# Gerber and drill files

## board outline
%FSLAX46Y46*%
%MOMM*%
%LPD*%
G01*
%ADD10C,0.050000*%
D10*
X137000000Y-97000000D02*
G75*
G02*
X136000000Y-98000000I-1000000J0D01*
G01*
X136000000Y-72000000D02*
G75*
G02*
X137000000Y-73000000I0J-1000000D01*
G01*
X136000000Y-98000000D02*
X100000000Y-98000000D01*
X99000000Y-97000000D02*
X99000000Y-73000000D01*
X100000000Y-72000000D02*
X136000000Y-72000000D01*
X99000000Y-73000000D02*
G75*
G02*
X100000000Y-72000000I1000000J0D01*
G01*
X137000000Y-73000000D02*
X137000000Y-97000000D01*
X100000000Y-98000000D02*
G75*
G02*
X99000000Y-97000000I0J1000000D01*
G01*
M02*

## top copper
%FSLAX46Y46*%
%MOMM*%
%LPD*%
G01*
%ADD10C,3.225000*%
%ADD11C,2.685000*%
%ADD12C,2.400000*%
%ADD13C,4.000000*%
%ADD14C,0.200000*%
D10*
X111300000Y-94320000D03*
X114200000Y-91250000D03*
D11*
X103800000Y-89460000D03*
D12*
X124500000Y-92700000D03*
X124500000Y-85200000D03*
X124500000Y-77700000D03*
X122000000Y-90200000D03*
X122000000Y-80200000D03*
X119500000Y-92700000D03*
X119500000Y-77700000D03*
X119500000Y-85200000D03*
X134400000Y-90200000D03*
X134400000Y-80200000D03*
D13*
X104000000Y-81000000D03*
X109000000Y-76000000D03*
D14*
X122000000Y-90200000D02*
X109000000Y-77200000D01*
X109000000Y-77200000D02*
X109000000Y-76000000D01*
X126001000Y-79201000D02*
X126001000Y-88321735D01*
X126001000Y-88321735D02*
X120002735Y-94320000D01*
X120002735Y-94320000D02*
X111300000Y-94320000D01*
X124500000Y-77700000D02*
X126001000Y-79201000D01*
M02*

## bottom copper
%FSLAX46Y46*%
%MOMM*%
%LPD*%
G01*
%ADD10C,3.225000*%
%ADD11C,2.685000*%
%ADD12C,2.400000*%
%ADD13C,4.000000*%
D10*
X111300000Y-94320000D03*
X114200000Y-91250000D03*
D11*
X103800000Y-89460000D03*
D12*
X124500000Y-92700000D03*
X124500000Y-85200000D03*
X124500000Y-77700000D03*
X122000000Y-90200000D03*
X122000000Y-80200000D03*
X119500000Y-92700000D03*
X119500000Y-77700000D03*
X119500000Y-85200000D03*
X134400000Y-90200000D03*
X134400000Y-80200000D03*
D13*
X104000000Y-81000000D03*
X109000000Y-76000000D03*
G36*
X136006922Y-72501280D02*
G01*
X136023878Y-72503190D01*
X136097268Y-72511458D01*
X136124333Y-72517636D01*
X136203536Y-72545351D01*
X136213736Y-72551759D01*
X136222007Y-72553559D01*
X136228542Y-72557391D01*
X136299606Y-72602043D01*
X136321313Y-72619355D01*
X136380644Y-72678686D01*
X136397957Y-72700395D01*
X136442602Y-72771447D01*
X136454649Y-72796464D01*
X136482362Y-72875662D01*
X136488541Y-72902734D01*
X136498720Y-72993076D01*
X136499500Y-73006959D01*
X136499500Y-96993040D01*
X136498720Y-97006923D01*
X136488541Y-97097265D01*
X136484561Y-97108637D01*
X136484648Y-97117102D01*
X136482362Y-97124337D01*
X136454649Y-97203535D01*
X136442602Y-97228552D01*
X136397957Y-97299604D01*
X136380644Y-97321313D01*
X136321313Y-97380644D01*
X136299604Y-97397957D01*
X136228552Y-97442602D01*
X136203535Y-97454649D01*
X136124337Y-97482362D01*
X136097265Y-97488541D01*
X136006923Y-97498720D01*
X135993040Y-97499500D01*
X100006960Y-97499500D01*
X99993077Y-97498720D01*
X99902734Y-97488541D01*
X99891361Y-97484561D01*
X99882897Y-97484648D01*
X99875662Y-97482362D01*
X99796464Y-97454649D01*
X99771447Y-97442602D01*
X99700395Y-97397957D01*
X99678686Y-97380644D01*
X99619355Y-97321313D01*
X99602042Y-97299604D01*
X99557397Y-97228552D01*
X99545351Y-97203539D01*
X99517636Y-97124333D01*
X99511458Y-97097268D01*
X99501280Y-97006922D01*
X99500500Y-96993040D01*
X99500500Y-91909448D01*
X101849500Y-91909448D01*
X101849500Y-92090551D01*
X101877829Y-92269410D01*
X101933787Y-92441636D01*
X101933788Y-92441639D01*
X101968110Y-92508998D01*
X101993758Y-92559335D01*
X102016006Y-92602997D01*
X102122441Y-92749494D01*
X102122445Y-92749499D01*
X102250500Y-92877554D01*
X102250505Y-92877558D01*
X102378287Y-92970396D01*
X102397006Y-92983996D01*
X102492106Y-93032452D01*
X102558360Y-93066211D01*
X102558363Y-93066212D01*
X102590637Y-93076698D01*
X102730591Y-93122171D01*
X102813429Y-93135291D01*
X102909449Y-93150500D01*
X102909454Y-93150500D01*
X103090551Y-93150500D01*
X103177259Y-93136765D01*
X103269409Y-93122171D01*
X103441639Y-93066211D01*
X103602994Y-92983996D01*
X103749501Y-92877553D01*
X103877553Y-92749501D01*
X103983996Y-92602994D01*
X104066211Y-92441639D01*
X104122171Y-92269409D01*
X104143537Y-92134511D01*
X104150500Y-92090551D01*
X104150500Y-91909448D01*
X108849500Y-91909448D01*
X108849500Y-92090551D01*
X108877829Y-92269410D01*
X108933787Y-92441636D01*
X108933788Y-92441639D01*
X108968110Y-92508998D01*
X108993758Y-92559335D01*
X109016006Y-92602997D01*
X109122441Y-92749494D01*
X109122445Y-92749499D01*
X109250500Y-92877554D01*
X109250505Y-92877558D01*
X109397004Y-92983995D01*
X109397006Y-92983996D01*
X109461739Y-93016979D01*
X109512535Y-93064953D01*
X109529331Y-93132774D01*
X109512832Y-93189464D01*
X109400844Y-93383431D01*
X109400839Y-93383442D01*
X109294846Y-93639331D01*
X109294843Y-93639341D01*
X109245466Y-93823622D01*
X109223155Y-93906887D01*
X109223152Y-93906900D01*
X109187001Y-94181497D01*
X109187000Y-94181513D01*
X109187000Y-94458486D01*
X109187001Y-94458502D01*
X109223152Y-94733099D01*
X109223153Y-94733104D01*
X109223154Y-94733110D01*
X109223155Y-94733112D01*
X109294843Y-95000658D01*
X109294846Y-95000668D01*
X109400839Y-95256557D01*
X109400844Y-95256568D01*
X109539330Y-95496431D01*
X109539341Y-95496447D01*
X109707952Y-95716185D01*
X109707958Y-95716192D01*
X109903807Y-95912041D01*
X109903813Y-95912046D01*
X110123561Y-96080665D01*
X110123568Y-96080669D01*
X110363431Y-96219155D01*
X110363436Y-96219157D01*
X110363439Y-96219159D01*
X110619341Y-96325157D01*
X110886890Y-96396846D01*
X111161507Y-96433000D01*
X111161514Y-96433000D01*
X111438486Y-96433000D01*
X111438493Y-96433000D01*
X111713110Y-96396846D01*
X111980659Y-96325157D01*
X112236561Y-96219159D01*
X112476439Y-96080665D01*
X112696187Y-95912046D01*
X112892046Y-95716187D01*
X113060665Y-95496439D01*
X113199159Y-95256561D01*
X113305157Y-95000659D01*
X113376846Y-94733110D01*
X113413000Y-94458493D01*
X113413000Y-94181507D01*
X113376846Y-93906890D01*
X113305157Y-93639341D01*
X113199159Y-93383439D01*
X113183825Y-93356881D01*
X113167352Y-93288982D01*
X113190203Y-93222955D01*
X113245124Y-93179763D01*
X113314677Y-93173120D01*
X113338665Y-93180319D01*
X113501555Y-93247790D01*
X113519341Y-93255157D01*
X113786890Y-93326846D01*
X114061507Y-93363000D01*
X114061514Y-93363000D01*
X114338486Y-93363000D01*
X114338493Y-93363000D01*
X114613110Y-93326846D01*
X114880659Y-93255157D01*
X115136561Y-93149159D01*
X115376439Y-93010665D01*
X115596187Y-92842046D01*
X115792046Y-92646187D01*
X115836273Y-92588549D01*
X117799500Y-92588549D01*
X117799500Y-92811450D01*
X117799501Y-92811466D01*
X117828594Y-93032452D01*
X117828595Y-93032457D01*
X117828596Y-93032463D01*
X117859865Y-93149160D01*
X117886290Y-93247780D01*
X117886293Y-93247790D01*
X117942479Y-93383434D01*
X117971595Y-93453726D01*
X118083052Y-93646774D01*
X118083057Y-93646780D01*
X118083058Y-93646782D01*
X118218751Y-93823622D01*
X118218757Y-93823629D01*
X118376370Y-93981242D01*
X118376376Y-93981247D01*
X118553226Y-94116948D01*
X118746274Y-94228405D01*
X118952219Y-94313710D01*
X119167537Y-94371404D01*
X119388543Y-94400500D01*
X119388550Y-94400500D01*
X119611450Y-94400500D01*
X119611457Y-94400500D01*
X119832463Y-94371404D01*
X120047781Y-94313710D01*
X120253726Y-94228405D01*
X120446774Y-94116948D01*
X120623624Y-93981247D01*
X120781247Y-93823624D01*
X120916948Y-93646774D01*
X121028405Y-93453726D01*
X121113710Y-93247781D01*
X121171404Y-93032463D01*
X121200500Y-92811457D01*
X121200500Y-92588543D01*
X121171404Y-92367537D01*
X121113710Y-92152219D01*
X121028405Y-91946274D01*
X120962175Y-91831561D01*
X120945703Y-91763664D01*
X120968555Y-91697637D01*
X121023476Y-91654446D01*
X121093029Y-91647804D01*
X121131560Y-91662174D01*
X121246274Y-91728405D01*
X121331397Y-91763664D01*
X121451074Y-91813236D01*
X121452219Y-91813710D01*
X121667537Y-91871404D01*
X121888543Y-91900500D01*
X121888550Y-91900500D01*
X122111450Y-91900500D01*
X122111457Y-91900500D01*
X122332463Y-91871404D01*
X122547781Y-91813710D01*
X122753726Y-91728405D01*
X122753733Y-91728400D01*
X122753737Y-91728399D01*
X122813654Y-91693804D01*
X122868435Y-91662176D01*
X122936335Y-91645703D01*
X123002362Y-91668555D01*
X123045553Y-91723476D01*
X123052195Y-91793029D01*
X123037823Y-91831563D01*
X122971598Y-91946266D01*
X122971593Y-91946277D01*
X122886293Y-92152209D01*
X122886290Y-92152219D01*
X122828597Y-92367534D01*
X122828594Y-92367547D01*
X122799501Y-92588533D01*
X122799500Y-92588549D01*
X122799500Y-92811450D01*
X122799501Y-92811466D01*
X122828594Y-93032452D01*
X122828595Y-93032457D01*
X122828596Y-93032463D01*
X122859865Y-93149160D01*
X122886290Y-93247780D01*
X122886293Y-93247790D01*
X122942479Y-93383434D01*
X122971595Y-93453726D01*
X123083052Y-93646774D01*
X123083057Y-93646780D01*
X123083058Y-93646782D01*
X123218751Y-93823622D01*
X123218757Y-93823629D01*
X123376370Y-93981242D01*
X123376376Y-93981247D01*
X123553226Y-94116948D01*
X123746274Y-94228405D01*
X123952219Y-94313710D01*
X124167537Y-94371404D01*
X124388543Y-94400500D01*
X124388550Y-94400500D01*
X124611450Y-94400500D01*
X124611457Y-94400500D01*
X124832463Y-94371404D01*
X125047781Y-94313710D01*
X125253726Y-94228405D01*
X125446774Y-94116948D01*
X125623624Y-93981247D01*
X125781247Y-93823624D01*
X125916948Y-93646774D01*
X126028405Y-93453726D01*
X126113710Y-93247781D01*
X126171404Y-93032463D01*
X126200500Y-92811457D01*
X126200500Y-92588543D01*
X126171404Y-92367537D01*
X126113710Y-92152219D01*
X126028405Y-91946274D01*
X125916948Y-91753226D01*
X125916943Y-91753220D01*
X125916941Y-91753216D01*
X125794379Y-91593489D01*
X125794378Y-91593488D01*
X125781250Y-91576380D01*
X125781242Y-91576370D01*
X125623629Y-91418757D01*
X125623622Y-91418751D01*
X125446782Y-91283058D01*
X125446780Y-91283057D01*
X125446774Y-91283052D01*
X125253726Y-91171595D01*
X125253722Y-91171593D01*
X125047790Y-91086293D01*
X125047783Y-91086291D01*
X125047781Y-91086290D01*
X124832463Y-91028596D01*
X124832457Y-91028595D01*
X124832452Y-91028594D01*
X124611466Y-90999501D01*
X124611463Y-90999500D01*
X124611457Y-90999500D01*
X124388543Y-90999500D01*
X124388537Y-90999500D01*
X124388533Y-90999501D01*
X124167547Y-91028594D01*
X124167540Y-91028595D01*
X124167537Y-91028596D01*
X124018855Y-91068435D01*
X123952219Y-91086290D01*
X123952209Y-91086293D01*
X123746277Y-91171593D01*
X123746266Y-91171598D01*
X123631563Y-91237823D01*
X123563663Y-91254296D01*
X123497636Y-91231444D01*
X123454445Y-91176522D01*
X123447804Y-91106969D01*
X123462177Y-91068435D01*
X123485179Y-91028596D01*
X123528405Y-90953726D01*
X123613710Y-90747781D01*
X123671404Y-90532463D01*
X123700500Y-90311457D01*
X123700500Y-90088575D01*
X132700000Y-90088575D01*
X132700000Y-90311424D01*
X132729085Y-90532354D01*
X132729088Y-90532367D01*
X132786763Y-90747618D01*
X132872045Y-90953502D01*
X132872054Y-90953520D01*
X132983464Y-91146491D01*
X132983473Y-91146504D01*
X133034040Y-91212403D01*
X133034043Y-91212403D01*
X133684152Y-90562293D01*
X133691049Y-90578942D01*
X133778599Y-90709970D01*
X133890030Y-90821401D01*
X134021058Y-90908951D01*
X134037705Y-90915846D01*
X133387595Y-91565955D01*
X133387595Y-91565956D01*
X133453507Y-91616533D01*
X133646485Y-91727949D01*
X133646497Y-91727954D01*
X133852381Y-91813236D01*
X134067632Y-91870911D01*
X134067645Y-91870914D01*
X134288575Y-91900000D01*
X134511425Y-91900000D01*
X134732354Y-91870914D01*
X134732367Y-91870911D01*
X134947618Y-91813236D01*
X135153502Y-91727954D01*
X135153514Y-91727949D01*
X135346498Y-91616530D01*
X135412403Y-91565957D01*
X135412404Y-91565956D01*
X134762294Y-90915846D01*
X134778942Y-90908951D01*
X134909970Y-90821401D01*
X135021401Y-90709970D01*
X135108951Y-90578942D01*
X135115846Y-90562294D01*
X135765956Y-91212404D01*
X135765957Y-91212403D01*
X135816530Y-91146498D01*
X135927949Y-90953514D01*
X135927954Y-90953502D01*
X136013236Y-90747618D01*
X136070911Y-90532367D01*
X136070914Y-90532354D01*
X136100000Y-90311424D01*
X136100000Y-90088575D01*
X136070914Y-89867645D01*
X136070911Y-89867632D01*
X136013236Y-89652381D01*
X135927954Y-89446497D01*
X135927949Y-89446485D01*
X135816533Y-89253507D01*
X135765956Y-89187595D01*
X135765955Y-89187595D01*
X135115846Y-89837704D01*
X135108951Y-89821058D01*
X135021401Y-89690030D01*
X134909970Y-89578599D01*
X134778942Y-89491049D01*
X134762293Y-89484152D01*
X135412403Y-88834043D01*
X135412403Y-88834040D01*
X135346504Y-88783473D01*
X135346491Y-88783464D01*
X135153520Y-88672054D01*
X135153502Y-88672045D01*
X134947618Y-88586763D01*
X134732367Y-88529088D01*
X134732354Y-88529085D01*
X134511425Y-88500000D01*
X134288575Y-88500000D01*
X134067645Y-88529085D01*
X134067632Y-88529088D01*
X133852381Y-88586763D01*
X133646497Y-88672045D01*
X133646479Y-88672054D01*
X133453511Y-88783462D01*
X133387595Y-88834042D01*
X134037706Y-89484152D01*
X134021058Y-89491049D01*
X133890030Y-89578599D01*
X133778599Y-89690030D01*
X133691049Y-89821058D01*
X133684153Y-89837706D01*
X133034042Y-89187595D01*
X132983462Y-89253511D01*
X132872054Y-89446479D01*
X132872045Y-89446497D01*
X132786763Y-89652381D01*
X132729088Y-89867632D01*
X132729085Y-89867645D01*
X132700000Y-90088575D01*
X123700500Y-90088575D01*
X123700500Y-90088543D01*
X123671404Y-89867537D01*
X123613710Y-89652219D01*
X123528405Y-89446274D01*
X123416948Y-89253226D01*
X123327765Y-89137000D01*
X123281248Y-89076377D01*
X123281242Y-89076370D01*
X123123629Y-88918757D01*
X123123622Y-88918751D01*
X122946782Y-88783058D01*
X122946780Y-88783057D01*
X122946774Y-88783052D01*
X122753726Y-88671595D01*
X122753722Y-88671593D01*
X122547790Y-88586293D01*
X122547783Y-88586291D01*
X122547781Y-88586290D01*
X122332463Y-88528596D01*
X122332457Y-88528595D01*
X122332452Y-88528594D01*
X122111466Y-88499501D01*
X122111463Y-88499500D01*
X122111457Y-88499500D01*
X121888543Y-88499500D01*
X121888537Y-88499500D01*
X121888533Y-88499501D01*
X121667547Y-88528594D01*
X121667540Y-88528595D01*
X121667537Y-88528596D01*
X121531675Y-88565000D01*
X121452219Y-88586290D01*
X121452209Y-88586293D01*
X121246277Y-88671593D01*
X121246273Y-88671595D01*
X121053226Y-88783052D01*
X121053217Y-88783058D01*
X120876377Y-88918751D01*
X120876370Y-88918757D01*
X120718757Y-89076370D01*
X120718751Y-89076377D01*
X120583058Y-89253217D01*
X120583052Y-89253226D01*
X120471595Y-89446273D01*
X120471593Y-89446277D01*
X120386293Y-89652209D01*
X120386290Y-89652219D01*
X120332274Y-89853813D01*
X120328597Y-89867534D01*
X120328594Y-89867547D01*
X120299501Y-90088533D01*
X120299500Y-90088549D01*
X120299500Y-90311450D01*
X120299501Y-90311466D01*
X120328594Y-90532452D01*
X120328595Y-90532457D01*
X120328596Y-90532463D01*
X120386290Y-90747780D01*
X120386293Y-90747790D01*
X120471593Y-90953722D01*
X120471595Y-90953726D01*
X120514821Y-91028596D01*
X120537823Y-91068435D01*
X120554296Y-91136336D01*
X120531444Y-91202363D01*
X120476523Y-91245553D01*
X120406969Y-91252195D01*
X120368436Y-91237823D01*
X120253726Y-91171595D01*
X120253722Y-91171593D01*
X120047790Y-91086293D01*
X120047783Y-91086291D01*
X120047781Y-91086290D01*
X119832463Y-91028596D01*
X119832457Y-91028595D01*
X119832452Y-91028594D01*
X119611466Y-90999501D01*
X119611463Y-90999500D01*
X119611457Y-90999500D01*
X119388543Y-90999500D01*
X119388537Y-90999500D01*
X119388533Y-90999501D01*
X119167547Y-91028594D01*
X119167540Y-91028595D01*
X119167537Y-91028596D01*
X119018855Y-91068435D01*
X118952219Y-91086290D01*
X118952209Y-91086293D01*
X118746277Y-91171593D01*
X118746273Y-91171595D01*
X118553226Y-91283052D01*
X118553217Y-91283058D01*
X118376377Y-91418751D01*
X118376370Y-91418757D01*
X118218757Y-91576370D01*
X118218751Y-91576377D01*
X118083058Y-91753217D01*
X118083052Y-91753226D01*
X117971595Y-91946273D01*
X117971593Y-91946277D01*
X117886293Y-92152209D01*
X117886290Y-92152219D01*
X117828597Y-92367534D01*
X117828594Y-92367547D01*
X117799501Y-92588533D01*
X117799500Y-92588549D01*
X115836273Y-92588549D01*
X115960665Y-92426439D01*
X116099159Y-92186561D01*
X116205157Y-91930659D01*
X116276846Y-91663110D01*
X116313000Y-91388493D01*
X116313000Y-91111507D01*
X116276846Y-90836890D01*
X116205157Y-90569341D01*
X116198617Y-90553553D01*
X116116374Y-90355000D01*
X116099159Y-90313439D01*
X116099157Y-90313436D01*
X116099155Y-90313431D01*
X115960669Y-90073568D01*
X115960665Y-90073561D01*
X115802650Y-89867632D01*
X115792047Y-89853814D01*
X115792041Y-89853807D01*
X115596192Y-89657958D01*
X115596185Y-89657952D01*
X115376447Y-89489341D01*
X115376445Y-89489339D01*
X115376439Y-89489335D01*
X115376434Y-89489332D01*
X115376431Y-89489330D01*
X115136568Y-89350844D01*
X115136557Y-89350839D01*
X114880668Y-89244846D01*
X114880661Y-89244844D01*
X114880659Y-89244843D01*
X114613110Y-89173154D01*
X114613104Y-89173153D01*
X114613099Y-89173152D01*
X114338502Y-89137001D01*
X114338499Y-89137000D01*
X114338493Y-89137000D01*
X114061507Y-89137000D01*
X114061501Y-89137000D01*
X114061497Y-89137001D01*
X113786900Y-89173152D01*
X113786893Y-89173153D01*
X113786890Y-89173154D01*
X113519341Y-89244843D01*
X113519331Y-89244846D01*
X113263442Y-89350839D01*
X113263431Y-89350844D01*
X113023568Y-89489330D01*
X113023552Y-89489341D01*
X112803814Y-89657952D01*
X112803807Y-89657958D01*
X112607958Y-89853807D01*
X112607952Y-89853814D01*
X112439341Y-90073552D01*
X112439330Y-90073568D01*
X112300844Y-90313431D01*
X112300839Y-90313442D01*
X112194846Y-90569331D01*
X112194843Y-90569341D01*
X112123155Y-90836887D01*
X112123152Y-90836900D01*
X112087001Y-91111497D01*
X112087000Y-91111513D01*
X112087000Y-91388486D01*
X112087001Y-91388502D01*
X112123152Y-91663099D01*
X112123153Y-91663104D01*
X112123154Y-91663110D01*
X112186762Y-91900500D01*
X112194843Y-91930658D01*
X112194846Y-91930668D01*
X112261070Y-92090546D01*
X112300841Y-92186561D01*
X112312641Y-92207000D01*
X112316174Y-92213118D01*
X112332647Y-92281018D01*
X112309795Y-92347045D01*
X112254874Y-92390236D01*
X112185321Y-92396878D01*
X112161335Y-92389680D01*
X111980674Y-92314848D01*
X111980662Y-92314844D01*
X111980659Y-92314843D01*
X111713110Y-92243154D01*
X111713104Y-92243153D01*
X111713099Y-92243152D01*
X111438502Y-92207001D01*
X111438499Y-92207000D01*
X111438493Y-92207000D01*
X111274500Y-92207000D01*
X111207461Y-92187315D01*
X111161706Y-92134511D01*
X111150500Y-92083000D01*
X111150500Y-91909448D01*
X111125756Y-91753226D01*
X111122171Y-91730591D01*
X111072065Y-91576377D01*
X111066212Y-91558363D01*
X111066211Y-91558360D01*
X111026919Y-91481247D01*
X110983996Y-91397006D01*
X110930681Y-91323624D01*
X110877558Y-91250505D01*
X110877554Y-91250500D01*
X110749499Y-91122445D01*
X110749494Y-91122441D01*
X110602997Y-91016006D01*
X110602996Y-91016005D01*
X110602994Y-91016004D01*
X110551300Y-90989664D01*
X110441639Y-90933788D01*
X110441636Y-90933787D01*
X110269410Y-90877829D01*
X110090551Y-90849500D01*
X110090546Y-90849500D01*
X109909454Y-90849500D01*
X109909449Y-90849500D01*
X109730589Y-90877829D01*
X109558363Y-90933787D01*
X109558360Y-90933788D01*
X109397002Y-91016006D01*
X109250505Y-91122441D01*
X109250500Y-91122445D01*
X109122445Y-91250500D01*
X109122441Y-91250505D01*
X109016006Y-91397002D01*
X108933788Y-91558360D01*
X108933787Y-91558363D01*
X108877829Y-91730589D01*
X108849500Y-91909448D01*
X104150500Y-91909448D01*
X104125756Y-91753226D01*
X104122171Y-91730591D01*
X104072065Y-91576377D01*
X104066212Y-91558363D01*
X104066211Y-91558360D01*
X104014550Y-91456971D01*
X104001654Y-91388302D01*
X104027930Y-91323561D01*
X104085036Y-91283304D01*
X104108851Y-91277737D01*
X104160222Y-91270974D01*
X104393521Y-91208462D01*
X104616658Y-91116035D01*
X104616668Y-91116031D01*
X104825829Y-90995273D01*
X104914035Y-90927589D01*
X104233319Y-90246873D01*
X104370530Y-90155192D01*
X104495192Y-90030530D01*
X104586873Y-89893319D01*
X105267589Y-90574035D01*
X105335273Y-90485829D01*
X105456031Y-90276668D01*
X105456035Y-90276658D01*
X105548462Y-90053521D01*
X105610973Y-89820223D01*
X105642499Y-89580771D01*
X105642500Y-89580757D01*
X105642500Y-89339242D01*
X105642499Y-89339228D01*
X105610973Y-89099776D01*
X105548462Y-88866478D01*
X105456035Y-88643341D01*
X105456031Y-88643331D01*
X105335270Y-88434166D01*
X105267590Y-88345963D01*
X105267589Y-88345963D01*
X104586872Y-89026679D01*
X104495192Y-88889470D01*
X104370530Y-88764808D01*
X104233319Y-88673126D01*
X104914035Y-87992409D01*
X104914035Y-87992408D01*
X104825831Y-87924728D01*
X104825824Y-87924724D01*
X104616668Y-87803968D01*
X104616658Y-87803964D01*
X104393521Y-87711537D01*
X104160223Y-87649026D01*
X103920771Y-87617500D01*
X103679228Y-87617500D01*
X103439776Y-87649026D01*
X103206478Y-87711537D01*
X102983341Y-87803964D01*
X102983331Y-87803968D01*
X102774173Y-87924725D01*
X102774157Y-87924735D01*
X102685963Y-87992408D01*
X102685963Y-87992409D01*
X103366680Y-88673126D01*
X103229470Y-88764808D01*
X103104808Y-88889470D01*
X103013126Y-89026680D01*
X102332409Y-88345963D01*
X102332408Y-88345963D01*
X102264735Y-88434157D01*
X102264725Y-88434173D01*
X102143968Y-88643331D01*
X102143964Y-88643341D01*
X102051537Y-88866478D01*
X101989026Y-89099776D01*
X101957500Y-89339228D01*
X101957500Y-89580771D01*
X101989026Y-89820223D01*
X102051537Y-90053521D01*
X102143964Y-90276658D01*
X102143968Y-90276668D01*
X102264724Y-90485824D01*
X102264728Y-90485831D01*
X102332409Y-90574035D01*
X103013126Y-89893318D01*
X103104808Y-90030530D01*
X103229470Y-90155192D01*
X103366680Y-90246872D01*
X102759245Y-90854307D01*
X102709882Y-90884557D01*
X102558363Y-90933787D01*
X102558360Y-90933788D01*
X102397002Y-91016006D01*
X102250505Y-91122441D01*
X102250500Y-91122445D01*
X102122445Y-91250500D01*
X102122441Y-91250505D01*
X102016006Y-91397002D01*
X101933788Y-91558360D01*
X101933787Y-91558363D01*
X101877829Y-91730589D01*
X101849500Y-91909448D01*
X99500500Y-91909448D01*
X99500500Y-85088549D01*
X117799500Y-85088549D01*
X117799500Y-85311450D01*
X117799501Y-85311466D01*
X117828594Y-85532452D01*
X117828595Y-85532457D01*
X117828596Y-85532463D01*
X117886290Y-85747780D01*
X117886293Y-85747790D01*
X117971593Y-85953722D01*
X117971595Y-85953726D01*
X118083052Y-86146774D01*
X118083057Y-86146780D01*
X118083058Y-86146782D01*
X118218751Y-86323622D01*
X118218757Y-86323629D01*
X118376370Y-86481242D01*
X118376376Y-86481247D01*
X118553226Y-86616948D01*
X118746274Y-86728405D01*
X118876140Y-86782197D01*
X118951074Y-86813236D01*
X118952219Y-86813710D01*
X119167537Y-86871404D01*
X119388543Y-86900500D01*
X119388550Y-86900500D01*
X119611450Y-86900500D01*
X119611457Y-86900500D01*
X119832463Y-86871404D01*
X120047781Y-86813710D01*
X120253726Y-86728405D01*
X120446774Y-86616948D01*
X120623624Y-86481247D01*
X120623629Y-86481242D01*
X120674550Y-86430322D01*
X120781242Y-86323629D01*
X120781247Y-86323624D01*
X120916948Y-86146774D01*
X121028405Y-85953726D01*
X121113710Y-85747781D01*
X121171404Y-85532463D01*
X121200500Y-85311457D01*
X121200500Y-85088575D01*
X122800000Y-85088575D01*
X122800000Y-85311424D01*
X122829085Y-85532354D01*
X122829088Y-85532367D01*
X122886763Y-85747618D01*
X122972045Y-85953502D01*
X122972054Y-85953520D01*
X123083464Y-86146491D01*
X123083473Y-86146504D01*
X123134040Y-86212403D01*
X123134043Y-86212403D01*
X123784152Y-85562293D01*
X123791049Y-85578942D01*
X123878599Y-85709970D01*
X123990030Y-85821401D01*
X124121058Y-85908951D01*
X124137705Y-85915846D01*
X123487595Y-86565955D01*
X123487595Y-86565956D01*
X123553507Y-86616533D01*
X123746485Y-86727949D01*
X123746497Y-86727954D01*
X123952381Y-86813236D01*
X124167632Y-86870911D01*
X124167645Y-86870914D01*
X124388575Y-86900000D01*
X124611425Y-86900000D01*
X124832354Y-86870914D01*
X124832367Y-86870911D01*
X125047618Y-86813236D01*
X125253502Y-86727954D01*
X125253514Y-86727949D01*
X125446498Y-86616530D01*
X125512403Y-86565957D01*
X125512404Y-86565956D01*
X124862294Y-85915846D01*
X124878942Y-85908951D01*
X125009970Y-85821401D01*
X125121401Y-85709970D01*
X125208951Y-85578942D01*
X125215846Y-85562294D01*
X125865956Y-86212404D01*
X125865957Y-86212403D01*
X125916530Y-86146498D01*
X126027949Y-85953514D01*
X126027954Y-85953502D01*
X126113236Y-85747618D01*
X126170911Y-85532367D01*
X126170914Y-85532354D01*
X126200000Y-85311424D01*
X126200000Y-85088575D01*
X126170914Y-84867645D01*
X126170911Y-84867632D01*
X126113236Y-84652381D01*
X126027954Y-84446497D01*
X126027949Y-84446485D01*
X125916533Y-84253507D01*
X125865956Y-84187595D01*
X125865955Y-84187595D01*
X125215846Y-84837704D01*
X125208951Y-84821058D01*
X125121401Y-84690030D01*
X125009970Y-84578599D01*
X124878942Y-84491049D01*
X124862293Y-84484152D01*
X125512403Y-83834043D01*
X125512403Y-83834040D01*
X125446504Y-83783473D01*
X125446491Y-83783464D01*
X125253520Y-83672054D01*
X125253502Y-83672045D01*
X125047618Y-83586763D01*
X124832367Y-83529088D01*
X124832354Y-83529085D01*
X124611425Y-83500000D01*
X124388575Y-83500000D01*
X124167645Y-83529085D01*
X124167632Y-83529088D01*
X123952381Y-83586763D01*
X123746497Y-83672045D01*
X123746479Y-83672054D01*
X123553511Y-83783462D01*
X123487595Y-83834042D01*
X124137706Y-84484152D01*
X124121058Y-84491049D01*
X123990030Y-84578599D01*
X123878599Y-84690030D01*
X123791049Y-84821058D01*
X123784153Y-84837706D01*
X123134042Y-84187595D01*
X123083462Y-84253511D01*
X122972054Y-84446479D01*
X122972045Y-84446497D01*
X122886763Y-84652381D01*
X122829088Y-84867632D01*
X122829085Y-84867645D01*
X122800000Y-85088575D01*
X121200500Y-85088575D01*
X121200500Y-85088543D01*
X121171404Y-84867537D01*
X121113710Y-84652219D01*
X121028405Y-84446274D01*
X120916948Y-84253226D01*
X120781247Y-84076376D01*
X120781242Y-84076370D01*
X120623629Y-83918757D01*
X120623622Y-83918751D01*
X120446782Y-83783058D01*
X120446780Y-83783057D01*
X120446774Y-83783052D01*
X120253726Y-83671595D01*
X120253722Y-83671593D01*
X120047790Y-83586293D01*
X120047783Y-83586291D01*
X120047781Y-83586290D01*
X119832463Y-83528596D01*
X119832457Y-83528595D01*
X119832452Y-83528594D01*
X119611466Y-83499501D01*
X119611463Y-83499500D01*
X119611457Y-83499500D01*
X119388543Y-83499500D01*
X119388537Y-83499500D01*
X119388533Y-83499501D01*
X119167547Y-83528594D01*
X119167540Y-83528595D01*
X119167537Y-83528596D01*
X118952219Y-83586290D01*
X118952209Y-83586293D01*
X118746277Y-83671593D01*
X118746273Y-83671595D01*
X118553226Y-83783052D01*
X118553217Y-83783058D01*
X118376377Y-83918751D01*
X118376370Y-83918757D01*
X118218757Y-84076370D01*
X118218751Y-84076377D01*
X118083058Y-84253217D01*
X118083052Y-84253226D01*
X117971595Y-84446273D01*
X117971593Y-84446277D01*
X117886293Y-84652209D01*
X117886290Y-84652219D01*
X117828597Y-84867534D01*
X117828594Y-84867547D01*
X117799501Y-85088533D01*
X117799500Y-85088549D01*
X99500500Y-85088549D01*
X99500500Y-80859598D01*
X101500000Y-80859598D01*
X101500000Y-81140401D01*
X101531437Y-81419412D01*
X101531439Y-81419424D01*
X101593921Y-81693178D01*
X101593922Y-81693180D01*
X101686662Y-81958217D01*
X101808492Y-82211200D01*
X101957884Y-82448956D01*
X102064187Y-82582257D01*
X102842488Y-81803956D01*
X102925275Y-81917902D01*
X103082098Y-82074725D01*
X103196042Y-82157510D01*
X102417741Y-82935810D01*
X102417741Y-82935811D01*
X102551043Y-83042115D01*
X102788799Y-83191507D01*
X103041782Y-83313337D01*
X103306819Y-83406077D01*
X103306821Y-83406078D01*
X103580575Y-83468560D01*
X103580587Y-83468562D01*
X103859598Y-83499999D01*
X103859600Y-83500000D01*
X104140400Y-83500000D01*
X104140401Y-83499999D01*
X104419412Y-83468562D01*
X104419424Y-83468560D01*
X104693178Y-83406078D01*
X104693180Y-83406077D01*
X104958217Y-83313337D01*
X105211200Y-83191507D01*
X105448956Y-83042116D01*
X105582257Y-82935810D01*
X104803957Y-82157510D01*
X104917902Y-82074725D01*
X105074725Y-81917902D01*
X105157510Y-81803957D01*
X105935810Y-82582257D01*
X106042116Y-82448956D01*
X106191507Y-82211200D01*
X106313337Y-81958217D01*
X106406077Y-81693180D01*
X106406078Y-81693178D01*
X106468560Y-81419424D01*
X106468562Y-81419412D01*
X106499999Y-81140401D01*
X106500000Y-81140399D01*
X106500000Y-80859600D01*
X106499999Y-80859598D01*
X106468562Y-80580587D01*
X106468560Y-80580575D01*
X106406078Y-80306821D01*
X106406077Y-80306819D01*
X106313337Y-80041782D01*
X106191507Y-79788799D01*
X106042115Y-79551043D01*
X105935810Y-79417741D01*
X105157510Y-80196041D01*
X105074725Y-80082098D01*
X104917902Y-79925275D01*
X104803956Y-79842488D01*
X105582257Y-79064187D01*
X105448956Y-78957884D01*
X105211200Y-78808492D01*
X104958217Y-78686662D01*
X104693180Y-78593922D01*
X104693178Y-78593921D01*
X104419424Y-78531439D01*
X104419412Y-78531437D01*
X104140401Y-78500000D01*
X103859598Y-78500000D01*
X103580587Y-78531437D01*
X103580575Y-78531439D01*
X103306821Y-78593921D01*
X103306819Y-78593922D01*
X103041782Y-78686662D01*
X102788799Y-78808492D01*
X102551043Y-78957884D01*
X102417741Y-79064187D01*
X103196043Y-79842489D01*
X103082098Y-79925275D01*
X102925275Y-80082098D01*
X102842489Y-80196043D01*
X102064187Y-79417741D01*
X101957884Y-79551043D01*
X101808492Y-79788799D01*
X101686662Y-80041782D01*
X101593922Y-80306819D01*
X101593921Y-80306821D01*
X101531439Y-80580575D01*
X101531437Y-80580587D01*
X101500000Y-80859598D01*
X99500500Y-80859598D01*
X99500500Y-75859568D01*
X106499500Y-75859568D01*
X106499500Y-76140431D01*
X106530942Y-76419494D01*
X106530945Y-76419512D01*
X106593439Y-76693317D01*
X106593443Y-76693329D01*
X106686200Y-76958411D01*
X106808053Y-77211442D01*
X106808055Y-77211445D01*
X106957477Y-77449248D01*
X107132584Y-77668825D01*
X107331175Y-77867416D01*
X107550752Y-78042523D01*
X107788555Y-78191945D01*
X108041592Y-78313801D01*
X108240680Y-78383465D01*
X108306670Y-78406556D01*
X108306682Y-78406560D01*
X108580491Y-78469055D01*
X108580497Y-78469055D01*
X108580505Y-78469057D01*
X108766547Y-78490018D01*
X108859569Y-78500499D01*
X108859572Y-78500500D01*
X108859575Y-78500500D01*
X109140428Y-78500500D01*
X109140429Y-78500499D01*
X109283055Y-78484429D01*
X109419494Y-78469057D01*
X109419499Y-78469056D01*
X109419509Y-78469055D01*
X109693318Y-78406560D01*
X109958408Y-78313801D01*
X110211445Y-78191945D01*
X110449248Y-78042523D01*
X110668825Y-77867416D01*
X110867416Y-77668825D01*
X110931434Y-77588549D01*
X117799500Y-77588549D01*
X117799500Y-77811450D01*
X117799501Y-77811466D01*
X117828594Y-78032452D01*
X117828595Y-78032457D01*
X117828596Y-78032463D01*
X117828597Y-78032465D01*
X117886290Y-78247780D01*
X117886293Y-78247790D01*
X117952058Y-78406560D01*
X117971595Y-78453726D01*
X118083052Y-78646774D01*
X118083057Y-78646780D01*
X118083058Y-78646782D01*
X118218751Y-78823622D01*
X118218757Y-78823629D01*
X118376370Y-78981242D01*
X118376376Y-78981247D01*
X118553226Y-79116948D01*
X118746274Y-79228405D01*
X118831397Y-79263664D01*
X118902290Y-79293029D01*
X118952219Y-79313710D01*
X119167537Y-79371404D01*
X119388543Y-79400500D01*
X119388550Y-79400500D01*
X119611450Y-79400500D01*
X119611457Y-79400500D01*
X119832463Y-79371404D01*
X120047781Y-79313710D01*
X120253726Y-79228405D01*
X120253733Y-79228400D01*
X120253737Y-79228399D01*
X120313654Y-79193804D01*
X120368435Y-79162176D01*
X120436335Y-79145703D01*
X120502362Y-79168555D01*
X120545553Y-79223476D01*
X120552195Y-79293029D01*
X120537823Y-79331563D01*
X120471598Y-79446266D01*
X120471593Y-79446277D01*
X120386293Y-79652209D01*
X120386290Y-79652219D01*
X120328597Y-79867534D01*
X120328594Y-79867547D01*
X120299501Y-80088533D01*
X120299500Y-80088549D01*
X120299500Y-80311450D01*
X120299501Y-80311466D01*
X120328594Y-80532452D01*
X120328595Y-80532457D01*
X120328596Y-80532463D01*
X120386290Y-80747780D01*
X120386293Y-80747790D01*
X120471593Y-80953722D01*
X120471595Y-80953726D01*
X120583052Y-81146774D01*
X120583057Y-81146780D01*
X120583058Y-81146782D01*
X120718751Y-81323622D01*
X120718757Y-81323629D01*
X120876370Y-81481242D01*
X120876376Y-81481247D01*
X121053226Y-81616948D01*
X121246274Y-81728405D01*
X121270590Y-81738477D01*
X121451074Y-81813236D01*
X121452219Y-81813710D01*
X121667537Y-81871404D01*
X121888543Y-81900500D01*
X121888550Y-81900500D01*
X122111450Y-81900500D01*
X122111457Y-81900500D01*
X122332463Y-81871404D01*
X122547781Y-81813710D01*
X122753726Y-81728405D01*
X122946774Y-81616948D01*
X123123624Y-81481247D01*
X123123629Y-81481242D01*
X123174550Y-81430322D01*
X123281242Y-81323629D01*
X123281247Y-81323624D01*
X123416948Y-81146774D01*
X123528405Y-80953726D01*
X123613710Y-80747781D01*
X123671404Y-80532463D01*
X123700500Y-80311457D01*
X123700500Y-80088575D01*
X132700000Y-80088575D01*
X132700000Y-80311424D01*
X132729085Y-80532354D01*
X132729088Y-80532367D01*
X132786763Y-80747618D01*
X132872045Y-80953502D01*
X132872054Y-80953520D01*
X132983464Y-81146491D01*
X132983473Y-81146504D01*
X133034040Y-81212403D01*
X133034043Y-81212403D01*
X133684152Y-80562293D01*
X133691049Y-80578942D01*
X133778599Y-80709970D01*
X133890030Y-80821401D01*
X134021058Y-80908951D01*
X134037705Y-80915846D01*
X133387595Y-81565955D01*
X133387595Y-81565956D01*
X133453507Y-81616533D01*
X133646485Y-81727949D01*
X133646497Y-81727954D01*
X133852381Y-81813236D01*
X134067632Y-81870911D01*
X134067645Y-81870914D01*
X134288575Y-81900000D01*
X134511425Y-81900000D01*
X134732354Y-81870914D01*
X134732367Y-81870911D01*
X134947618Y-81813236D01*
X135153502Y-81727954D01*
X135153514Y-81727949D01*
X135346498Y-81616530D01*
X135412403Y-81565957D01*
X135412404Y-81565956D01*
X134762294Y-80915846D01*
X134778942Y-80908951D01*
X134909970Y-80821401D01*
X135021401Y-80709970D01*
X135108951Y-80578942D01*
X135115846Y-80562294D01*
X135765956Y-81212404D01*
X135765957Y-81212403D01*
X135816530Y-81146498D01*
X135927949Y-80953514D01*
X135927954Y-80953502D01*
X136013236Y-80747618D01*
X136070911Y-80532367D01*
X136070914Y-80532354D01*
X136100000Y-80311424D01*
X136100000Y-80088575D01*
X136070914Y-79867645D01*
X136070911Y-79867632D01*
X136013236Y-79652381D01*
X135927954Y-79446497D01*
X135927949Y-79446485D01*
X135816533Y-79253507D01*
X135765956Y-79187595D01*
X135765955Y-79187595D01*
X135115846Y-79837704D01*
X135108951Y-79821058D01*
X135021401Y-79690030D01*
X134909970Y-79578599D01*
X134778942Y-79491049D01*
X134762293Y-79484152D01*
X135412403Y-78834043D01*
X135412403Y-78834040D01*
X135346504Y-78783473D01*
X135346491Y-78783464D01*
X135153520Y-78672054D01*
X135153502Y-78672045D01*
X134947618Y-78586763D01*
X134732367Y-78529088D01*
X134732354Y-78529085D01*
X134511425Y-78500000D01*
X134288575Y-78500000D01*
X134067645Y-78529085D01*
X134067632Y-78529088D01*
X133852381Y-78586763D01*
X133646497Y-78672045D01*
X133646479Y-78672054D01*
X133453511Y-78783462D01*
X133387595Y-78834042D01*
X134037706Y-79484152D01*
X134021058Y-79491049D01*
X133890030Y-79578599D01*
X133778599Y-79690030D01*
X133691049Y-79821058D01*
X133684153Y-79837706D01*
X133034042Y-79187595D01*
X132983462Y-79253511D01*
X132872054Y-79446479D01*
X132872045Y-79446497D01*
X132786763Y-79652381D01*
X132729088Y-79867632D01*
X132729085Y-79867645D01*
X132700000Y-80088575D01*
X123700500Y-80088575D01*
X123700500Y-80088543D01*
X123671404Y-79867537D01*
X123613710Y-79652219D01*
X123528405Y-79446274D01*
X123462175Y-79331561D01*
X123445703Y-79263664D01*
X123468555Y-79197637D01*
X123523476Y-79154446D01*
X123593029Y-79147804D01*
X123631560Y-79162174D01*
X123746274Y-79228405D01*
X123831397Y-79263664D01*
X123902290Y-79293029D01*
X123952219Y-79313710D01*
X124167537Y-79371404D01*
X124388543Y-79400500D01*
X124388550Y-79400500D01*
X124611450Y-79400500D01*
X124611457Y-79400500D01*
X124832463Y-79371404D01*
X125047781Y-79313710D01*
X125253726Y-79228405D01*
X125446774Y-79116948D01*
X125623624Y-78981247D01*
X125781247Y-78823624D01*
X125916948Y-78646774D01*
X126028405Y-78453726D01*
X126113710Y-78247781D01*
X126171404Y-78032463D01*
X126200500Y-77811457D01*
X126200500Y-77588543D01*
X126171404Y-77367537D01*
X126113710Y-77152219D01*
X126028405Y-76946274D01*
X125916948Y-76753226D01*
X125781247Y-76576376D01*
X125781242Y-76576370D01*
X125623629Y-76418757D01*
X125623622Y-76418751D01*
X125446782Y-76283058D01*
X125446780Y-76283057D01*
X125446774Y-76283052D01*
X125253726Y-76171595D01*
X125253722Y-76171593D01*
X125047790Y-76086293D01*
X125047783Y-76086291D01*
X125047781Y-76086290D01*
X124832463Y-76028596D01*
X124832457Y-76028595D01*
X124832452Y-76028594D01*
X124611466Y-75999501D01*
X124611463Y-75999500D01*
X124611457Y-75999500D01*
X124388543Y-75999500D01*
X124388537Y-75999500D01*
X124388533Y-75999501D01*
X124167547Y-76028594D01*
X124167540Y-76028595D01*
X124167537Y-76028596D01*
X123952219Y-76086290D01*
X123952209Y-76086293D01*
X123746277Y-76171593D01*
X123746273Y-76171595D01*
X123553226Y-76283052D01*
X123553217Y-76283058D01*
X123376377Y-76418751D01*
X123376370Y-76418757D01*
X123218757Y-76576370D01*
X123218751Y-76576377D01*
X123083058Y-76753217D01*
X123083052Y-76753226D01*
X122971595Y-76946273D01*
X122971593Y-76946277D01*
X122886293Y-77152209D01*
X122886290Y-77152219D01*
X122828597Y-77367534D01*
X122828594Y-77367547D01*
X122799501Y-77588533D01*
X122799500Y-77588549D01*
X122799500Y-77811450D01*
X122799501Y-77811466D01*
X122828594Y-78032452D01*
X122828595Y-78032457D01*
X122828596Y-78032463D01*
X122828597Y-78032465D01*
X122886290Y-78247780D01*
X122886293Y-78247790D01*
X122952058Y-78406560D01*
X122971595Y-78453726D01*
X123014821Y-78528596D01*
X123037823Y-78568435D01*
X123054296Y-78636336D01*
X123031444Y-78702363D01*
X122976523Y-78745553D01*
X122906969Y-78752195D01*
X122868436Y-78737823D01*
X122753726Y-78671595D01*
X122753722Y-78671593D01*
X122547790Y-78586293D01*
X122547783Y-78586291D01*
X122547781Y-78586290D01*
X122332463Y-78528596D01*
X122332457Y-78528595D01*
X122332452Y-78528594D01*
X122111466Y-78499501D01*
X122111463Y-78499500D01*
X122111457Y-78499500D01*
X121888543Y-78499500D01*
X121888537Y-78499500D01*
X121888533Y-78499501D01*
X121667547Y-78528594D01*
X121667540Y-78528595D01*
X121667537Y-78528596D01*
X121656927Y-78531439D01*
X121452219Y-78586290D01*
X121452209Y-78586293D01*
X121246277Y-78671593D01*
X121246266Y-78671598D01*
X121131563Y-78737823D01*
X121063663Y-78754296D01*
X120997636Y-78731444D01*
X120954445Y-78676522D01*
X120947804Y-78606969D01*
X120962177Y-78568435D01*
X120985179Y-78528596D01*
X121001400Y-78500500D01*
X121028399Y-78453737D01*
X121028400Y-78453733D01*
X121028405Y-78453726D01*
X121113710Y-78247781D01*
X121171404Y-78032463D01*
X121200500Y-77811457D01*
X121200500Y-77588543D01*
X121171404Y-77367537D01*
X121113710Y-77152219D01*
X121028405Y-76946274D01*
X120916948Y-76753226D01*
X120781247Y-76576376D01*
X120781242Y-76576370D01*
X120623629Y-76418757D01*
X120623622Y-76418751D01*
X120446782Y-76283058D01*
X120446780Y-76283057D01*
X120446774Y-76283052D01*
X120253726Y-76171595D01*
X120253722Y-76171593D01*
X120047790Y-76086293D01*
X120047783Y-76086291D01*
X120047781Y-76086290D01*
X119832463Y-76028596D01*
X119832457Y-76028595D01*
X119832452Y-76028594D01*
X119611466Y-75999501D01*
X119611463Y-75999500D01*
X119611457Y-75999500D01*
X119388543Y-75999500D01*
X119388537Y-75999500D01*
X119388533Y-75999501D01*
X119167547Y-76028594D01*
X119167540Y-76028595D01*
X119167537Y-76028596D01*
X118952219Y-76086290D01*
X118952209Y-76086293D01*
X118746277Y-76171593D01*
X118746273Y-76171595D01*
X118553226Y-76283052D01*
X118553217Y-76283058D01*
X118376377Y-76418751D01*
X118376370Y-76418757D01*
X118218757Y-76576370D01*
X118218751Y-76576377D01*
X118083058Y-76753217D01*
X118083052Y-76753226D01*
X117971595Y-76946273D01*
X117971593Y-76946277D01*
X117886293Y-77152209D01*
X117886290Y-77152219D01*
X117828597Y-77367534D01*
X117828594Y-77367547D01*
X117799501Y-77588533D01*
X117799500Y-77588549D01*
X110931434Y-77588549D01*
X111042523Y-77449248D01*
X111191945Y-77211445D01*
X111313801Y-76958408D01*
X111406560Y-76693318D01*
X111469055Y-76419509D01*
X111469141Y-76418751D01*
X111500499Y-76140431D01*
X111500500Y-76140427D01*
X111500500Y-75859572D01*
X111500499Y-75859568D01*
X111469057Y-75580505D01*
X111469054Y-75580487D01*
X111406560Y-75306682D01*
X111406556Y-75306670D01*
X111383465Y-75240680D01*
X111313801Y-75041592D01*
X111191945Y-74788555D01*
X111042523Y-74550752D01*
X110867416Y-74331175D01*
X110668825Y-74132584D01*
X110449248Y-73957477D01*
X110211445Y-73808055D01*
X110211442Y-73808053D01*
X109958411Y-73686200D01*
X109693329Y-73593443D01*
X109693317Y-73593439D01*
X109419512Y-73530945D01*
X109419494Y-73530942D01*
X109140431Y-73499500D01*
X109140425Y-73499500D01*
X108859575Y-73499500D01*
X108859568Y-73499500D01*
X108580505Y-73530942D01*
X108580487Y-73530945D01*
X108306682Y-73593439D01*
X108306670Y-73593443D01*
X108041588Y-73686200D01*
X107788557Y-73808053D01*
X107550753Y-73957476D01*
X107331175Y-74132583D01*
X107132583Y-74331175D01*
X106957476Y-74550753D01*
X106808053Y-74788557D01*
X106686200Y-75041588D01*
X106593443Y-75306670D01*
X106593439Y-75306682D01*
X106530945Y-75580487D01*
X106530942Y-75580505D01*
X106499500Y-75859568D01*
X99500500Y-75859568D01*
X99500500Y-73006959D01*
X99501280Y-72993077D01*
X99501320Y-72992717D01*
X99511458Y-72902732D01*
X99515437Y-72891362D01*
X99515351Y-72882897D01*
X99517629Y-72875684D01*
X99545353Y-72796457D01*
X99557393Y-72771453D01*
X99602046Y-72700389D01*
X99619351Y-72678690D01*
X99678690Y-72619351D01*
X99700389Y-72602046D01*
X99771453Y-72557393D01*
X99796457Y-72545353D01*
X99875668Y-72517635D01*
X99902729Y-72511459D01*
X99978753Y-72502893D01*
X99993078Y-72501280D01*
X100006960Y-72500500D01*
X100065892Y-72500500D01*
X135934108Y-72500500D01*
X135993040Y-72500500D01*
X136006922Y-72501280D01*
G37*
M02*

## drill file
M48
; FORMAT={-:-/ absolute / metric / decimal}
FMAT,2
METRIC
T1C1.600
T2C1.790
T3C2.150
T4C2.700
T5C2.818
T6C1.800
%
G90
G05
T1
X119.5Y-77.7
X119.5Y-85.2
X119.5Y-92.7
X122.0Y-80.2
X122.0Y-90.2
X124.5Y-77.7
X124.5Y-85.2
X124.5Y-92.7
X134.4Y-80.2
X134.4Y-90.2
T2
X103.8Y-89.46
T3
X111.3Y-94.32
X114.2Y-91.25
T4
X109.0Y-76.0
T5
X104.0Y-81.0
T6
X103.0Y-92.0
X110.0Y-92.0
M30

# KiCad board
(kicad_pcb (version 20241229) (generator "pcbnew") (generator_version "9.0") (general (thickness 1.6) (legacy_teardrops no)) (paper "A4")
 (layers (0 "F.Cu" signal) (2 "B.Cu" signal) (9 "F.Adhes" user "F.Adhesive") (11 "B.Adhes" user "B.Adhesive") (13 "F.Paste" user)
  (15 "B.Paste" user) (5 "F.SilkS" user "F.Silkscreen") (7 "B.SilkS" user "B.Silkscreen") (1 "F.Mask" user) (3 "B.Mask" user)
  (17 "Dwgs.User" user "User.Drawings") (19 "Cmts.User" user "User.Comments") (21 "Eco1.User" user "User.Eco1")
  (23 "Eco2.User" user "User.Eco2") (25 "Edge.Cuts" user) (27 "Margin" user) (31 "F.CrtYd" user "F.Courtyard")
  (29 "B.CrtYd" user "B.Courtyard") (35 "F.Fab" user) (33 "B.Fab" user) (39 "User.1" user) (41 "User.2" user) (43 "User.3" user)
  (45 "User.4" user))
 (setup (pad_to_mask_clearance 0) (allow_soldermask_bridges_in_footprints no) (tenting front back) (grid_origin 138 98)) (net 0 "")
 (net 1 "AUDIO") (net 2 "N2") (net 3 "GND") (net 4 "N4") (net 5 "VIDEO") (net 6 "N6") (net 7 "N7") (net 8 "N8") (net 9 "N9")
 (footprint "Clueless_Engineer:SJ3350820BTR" (layer "F.Cu") (at 111.3 94.32)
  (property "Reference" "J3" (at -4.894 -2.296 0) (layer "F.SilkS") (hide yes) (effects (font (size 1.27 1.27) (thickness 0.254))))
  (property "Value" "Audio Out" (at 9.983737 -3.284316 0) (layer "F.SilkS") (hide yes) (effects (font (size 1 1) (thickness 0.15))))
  (pad "" np_thru_hole circle (at -8.3 -2.32) (size 1.8 1.8) (drill 1.8) (layers "*.Cu" "*.Mask"))
  (pad "" np_thru_hole circle (at -1.3 -2.32) (size 1.8 1.8) (drill 1.8) (layers "*.Cu" "*.Mask"))
  (pad "2" thru_hole circle (at 0 0) (size 3.225 3.225) (drill 2.15) (layers "*.Cu" "*.Mask") (remove_unused_layers no) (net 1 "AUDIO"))
  (pad "3" thru_hole circle (at 2.9 -3.07) (size 3.225 3.225) (drill 2.15) (layers "*.Cu" "*.Mask") (remove_unused_layers no) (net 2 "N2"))
  (pad "5" thru_hole circle (at -7.5 -4.86) (size 2.685 2.685) (drill 1.79) (layers "*.Cu" "*.Mask") (remove_unused_layers no) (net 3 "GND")))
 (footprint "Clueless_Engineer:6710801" (layer "F.Cu") (at 124.5 92.7 -90)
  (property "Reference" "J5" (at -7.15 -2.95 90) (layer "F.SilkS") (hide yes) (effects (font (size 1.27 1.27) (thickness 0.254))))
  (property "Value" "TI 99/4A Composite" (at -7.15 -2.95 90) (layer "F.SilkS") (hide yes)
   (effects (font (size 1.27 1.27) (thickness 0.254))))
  (pad "1" thru_hole circle (at 0 0 270) (size 2.4 2.4) (drill 1.6) (layers "*.Cu" "*.Mask") (remove_unused_layers no) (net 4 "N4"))
  (pad "2" thru_hole circle (at -7.5 0 270) (size 2.4 2.4) (drill 1.6) (layers "*.Cu" "*.Mask") (remove_unused_layers no) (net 3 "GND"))
  (pad "3" thru_hole circle (at -15 0 270) (size 2.4 2.4) (drill 1.6) (layers "*.Cu" "*.Mask") (remove_unused_layers no) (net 1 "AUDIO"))
  (pad "4" thru_hole circle (at -2.5 2.5 270) (size 2.4 2.4) (drill 1.6) (layers "*.Cu" "*.Mask") (remove_unused_layers no) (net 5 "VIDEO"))
  (pad "5" thru_hole circle (at -12.5 2.5 270) (size 2.4 2.4) (drill 1.6) (layers "*.Cu" "*.Mask") (remove_unused_layers no) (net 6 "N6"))
  (pad "6" thru_hole circle (at 0 5 270) (size 2.4 2.4) (drill 1.6) (layers "*.Cu" "*.Mask") (remove_unused_layers no) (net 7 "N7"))
  (pad "7" thru_hole circle (at -15 5 270) (size 2.4 2.4) (drill 1.6) (layers "*.Cu" "*.Mask") (remove_unused_layers no) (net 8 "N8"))
  (pad "8" thru_hole circle (at -7.5 5 270) (size 2.4 2.4) (drill 1.6) (layers "*.Cu" "*.Mask") (remove_unused_layers no) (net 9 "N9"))
  (pad "MH1" thru_hole circle (at -2.5 -9.9 270) (size 2.4 2.4) (drill 1.6) (layers "*.Cu" "*.Mask") (remove_unused_layers no) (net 3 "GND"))
  (pad "MH2" thru_hole circle (at -12.5 -9.9 270) (size 2.4 2.4) (drill 1.6) (layers "*.Cu" "*.Mask") (remove_unused_layers no)
   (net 3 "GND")))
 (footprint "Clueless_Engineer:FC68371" (layer "F.Cu") (at 104 81)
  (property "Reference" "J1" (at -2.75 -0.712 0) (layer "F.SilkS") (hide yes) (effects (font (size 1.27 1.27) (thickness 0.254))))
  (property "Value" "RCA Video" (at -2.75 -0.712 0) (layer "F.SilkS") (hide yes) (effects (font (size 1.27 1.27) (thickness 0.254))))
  (pad "1" thru_hole circle (at 0 0) (size 4 4) (drill 2.818) (layers "*.Cu" "*.Mask") (remove_unused_layers no) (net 3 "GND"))
  (pad "3" thru_hole circle (at 5 -5) (size 4 4) (drill 2.7) (layers "*.Cu" "*.Mask") (remove_unused_layers no) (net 5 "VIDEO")))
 (gr_arc (start 137 97) (mid 136.707107 97.707107) (end 136 98) (stroke (width 0.05) (type default)) (layer "Edge.Cuts"))
 (gr_arc (start 136 72) (mid 136.707107 72.292893) (end 137 73) (stroke (width 0.05) (type default)) (layer "Edge.Cuts"))
 (gr_line (start 136 98) (end 100 98) (stroke (width 0.05) (type default)) (layer "Edge.Cuts"))
 (gr_line (start 99 97) (end 99 73) (stroke (width 0.05) (type default)) (layer "Edge.Cuts"))
 (gr_line (start 100 72) (end 136 72) (stroke (width 0.05) (type default)) (layer "Edge.Cuts"))
 (gr_arc (start 99 73) (mid 99.292893 72.292893) (end 100 72) (stroke (width 0.05) (type default)) (layer "Edge.Cuts"))
 (gr_line (start 137 73) (end 137 97) (stroke (width 0.05) (type default)) (layer "Edge.Cuts"))
 (gr_arc (start 100 98) (mid 99.292893 97.707107) (end 99 97) (stroke (width 0.05) (type default)) (layer "Edge.Cuts"))
 (segment (start 122 90.2) (end 109 77.2) (width 0.2) (layer "F.Cu") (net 5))
 (segment (start 109 77.2) (end 109 76) (width 0.2) (layer "F.Cu") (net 5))
 (segment (start 126.001 79.201) (end 126.001 88.321735) (width 0.2) (layer "F.Cu") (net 1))
 (segment (start 126.001 88.321735) (end 120.002735 94.32) (width 0.2) (layer "F.Cu") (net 1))
 (segment (start 120.002735 94.32) (end 111.3 94.32) (width 0.2) (layer "F.Cu") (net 1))
 (segment (start 124.5 77.7) (end 126.001 79.201) (width 0.2) (layer "F.Cu") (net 1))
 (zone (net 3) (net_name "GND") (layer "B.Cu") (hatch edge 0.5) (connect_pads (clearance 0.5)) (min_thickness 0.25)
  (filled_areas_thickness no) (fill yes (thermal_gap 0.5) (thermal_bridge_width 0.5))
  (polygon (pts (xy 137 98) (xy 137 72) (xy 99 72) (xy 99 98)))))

